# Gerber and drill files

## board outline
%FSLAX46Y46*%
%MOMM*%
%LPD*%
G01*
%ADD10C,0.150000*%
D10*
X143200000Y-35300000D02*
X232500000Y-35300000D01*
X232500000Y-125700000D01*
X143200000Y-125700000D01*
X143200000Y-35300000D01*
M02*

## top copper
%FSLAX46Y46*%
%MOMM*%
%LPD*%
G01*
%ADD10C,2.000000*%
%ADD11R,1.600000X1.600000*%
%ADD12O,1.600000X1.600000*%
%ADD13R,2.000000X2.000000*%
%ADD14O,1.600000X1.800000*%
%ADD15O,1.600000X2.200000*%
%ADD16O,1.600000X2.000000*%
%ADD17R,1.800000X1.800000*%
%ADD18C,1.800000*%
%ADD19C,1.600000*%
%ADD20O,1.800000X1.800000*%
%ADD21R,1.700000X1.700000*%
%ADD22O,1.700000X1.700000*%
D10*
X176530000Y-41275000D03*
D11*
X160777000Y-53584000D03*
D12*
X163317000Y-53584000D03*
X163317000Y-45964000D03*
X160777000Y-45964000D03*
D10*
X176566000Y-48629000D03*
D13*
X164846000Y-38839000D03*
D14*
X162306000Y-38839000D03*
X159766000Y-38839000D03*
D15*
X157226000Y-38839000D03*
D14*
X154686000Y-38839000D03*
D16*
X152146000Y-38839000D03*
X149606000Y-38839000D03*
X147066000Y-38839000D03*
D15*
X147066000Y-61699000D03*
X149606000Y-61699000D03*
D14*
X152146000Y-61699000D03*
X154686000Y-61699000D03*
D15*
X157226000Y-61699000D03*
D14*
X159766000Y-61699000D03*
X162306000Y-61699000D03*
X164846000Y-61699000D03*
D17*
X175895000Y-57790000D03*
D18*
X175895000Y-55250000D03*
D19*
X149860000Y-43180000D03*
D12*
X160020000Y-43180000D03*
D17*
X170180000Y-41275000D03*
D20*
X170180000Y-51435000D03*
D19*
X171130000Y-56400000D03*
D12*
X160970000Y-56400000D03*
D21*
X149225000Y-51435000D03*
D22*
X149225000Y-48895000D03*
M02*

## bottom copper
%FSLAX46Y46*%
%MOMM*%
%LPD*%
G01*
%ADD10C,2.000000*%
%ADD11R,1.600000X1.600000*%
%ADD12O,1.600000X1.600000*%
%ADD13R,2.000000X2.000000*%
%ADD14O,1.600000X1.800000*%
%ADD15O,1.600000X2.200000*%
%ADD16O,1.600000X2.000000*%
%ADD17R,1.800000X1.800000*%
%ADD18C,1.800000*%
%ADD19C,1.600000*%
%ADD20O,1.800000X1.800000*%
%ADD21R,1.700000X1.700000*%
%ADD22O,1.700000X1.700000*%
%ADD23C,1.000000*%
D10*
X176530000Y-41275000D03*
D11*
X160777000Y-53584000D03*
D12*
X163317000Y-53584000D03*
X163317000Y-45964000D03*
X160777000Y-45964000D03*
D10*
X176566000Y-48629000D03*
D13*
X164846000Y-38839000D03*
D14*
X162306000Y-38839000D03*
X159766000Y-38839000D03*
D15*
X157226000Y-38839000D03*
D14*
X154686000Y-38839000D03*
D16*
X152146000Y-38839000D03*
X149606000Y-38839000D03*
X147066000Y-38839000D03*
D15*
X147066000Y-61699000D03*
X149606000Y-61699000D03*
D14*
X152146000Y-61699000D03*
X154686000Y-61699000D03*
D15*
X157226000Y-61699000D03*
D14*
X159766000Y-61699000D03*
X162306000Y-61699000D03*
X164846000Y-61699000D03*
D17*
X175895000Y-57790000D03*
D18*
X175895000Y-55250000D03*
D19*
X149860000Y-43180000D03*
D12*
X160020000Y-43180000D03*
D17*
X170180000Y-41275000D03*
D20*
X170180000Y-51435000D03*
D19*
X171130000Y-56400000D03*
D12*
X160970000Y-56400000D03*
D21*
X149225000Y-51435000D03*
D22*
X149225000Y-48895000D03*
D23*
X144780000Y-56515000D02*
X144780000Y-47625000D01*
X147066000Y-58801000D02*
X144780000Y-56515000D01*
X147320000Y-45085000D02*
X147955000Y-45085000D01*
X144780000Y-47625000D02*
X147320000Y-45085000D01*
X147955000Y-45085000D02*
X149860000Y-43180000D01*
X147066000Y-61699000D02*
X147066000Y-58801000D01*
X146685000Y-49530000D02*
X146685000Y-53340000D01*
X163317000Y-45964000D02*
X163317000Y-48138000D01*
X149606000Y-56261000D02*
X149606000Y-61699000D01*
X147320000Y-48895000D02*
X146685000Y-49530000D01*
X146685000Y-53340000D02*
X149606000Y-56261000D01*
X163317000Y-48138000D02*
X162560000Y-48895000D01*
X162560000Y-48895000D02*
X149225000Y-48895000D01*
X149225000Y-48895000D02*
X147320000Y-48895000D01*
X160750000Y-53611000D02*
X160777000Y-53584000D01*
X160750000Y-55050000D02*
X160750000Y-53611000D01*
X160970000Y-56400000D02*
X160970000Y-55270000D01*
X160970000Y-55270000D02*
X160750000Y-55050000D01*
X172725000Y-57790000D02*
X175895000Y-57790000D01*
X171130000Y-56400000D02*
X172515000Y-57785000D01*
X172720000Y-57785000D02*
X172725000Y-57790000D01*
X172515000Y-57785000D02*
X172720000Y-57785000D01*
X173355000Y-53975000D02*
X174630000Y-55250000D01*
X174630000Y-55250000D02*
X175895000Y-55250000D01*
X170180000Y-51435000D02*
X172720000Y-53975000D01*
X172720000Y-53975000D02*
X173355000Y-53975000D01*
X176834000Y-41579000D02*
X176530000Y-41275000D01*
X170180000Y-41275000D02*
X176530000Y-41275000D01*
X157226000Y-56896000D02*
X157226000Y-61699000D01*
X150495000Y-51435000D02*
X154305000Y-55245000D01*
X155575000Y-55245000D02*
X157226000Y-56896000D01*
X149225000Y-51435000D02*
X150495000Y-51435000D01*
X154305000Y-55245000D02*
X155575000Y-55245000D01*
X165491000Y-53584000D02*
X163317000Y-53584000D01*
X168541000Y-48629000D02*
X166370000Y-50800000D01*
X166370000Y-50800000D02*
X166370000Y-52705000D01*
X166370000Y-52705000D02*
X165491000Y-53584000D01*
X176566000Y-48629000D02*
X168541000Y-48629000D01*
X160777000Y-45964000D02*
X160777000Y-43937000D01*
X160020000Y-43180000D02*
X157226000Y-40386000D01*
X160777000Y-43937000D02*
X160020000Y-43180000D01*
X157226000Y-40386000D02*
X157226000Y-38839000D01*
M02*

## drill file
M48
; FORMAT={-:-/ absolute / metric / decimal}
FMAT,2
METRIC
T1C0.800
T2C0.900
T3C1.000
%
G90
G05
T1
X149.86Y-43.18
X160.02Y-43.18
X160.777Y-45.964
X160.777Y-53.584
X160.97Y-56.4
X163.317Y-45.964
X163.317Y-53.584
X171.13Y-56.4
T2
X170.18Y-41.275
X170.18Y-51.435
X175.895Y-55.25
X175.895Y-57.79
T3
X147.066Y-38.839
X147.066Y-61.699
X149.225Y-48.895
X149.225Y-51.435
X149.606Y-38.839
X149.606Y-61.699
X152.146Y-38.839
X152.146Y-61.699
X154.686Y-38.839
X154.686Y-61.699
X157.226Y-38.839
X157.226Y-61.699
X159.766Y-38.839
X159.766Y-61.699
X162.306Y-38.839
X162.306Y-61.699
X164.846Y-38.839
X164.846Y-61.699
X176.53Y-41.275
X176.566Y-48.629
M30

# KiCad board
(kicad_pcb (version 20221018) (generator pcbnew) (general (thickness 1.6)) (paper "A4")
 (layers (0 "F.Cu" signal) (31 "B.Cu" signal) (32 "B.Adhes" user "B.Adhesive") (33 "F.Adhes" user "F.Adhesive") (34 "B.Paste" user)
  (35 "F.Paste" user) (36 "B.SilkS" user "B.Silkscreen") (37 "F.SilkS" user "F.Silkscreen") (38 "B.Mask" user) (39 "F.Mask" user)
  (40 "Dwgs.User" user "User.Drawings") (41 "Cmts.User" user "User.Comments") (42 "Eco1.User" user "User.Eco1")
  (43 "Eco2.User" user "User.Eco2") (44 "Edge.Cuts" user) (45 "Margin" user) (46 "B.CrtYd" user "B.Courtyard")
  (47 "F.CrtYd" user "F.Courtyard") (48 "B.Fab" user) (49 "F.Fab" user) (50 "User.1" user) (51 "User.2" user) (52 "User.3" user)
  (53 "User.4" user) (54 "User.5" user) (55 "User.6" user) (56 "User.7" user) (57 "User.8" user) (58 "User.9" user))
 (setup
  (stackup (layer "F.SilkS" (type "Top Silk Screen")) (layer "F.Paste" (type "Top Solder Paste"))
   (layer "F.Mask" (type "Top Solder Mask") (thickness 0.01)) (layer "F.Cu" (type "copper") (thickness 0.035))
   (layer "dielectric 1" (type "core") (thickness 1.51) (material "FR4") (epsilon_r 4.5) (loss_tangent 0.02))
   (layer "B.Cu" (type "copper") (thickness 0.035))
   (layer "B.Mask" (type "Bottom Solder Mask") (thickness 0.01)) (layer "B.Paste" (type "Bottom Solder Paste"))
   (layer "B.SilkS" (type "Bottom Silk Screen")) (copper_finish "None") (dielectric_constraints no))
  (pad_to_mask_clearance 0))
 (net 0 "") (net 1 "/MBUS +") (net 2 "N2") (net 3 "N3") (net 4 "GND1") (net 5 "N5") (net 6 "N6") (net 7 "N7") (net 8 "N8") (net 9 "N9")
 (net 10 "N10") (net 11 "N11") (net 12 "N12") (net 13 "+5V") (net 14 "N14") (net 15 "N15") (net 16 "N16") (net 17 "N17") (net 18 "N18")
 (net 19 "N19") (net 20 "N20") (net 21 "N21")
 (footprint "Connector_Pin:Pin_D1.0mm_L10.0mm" (layer "F.Cu") (at 176.53 41.275 180)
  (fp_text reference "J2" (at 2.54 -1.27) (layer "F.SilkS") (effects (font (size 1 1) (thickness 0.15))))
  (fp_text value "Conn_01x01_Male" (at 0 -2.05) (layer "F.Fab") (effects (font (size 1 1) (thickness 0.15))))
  (pad "1" thru_hole circle (at 0 0 180) (size 2 2) (drill 1) (layers "*.Cu" "*.Mask") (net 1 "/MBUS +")))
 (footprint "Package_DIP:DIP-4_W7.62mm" (layer "F.Cu") (at 160.777 53.584 90)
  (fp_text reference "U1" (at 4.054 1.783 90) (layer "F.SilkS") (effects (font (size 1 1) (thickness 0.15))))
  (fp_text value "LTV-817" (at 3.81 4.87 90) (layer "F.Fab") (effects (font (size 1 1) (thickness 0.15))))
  (pad "1" thru_hole rect (at 0 0 90) (size 1.6 1.6) (drill 0.8) (layers "*.Cu" "*.Mask") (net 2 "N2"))
  (pad "2" thru_hole oval (at 0 2.54 90) (size 1.6 1.6) (drill 0.8) (layers "*.Cu" "*.Mask") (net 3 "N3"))
  (pad "3" thru_hole oval (at 7.62 2.54 90) (size 1.6 1.6) (drill 0.8) (layers "*.Cu" "*.Mask") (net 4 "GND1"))
  (pad "4" thru_hole oval (at 7.62 0 90) (size 1.6 1.6) (drill 0.8) (layers "*.Cu" "*.Mask") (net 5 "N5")))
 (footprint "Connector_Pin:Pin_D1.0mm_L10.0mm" (layer "F.Cu") (at 176.566 48.629 180)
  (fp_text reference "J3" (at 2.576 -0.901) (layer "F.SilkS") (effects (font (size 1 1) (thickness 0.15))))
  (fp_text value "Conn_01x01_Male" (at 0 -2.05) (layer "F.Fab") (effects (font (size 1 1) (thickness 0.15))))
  (pad "1" thru_hole circle (at 0 0 180) (size 2 2) (drill 1) (layers "*.Cu" "*.Mask") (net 3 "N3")))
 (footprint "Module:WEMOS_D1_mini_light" (layer "F.Cu") (at 164.846 38.839 -90)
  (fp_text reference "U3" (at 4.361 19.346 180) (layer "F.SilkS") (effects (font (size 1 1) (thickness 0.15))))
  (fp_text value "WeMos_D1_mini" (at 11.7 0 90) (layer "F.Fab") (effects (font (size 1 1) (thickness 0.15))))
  (pad "1" thru_hole rect (at 0 0 270) (size 2 2) (drill 1) (layers "*.Cu" "*.Mask") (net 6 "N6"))
  (pad "2" thru_hole oval (at 0 2.54 270) (size 1.8 1.6) (drill 1) (layers "*.Cu" "*.Mask") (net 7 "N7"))
  (pad "3" thru_hole oval (at 0 5.08 270) (size 1.8 1.6) (drill 1) (layers "*.Cu" "*.Mask") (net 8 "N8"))
  (pad "4" thru_hole oval (at 0 7.62 270) (size 2.2 1.6) (drill 1) (layers "*.Cu" "*.Mask") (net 5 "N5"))
  (pad "5" thru_hole oval (at 0 10.16 270) (size 1.8 1.6) (drill 1) (layers "*.Cu" "*.Mask") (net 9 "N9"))
  (pad "6" thru_hole oval (at 0 12.7 270) (size 2 1.6) (drill 1) (layers "*.Cu" "*.Mask") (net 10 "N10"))
  (pad "7" thru_hole oval (at 0 15.24 270) (size 2 1.6) (drill 1) (layers "*.Cu" "*.Mask") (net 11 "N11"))
  (pad "8" thru_hole oval (at 0 17.78 270) (size 2 1.6) (drill 1) (layers "*.Cu" "*.Mask") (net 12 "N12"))
  (pad "9" thru_hole oval (at 22.86 17.78 270) (size 2.2 1.6) (drill 1) (layers "*.Cu" "*.Mask") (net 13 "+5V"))
  (pad "10" thru_hole oval (at 22.86 15.24 270) (size 2.2 1.6) (drill 1) (layers "*.Cu" "*.Mask") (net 4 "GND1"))
  (pad "11" thru_hole oval (at 22.86 12.7 270) (size 1.8 1.6) (drill 1) (layers "*.Cu" "*.Mask") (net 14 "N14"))
  (pad "12" thru_hole oval (at 22.86 10.16 270) (size 1.8 1.6) (drill 1) (layers "*.Cu" "*.Mask") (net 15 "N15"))
  (pad "13" thru_hole oval (at 22.86 7.62 270) (size 2.2 1.6) (drill 1) (layers "*.Cu" "*.Mask") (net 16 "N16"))
  (pad "14" thru_hole oval (at 22.86 5.08 270) (size 1.8 1.6) (drill 1) (layers "*.Cu" "*.Mask") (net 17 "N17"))
  (pad "15" thru_hole oval (at 22.86 2.54 270) (size 1.8 1.6) (drill 1) (layers "*.Cu" "*.Mask") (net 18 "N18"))
  (pad "16" thru_hole oval (at 22.86 0 270) (size 1.8 1.6) (drill 1) (layers "*.Cu" "*.Mask") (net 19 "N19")))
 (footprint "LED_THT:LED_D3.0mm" (layer "F.Cu") (at 175.895 57.79 90)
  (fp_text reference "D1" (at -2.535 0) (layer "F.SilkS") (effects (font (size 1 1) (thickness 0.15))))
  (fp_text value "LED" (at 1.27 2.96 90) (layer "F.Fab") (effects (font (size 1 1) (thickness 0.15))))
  (pad "1" thru_hole rect (at 0 0 90) (size 1.8 1.8) (drill 0.9) (layers "*.Cu" "*.Mask") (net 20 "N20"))
  (pad "2" thru_hole circle (at 2.54 0 90) (size 1.8 1.8) (drill 0.9) (layers "*.Cu" "*.Mask") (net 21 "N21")))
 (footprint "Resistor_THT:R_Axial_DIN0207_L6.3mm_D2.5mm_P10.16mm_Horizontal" (layer "F.Cu") (at 149.86 43.18)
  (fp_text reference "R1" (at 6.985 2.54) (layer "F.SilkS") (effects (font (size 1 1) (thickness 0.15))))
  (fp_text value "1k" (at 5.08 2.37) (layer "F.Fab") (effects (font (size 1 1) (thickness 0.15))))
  (pad "1" thru_hole circle (at 0 0) (size 1.6 1.6) (drill 0.8) (layers "*.Cu" "*.Mask") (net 13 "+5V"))
  (pad "2" thru_hole oval (at 10.16 0) (size 1.6 1.6) (drill 0.8) (layers "*.Cu" "*.Mask") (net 5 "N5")))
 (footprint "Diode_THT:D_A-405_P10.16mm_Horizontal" (layer "F.Cu") (at 170.18 41.275 -90)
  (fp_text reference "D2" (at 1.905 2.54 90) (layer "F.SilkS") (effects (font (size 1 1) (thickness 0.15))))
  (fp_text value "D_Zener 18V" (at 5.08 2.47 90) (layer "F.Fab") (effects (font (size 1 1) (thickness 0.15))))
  (pad "1" thru_hole rect (at 0 0 270) (size 1.8 1.8) (drill 0.9) (layers "*.Cu" "*.Mask") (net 1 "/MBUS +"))
  (pad "2" thru_hole oval (at 10.16 0 270) (size 1.8 1.8) (drill 0.9) (layers "*.Cu" "*.Mask") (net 21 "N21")))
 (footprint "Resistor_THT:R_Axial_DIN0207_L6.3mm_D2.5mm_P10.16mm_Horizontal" (layer "F.Cu") (at 171.13 56.4 180)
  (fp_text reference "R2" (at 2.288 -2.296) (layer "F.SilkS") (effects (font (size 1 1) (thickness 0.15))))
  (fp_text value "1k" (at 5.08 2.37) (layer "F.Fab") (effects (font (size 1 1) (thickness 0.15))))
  (pad "1" thru_hole circle (at 0 0 180) (size 1.6 1.6) (drill 0.8) (layers "*.Cu" "*.Mask") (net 20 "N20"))
  (pad "2" thru_hole oval (at 10.16 0 180) (size 1.6 1.6) (drill 0.8) (layers "*.Cu" "*.Mask") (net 2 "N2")))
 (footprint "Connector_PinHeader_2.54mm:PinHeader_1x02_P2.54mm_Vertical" (layer "F.Cu") (at 149.225 51.435 180)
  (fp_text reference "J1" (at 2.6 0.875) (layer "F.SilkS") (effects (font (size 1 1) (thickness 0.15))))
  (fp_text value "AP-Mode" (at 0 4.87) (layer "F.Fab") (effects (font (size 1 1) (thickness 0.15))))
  (pad "1" thru_hole rect (at 0 0 180) (size 1.7 1.7) (drill 1) (layers "*.Cu" "*.Mask") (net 16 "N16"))
  (pad "2" thru_hole oval (at 0 2.54 180) (size 1.7 1.7) (drill 1) (layers "*.Cu" "*.Mask") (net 4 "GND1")))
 (gr_rect (start 143.2 35.3) (end 232.5 125.7) (stroke (width 0.15) (type solid)) (fill none) (layer "Edge.Cuts"))
 (segment (start 144.78 56.515) (end 144.78 47.625) (width 1) (layer "B.Cu") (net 13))
 (segment (start 147.066 58.801) (end 144.78 56.515) (width 1) (layer "B.Cu") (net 13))
 (segment (start 147.32 45.085) (end 147.955 45.085) (width 1) (layer "B.Cu") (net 13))
 (segment (start 144.78 47.625) (end 147.32 45.085) (width 1) (layer "B.Cu") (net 13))
 (segment (start 147.955 45.085) (end 149.86 43.18) (width 1) (layer "B.Cu") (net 13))
 (segment (start 147.066 61.699) (end 147.066 58.801) (width 1) (layer "B.Cu") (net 13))
 (segment (start 146.685 49.53) (end 146.685 53.34) (width 1) (layer "B.Cu") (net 4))
 (segment (start 163.317 45.964) (end 163.317 48.138) (width 1) (layer "B.Cu") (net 4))
 (segment (start 149.606 56.261) (end 149.606 61.699) (width 1) (layer "B.Cu") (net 4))
 (segment (start 147.32 48.895) (end 146.685 49.53) (width 1) (layer "B.Cu") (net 4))
 (segment (start 146.685 53.34) (end 149.606 56.261) (width 1) (layer "B.Cu") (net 4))
 (segment (start 163.317 48.138) (end 162.56 48.895) (width 1) (layer "B.Cu") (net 4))
 (segment (start 162.56 48.895) (end 149.225 48.895) (width 1) (layer "B.Cu") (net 4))
 (segment (start 149.225 48.895) (end 147.32 48.895) (width 1) (layer "B.Cu") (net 4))
 (segment (start 160.75 53.611) (end 160.777 53.584) (width 1) (layer "B.Cu") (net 2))
 (segment (start 160.75 55.05) (end 160.75 53.611) (width 1) (layer "B.Cu") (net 2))
 (segment (start 160.97 56.4) (end 160.97 55.27) (width 1) (layer "B.Cu") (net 2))
 (segment (start 160.97 55.27) (end 160.75 55.05) (width 1) (layer "B.Cu") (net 2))
 (segment (start 172.725 57.79) (end 175.895 57.79) (width 1) (layer "B.Cu") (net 20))
 (segment (start 171.13 56.4) (end 172.515 57.785) (width 1) (layer "B.Cu") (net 20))
 (segment (start 172.72 57.785) (end 172.725 57.79) (width 1) (layer "B.Cu") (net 20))
 (segment (start 172.515 57.785) (end 172.72 57.785) (width 1) (layer "B.Cu") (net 20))
 (segment (start 173.355 53.975) (end 174.63 55.25) (width 1) (layer "B.Cu") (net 21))
 (segment (start 174.63 55.25) (end 175.895 55.25) (width 1) (layer "B.Cu") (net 21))
 (segment (start 170.18 51.435) (end 172.72 53.975) (width 1) (layer "B.Cu") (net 21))
 (segment (start 172.72 53.975) (end 173.355 53.975) (width 1) (layer "B.Cu") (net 21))
 (segment (start 176.834 41.579) (end 176.53 41.275) (width 1) (layer "B.Cu") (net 1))
 (segment (start 170.18 41.275) (end 176.53 41.275) (width 1) (layer "B.Cu") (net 1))
 (segment (start 157.226 56.896) (end 157.226 61.699) (width 1) (layer "B.Cu") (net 16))
 (segment (start 150.495 51.435) (end 154.305 55.245) (width 1) (layer "B.Cu") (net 16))
 (segment (start 155.575 55.245) (end 157.226 56.896) (width 1) (layer "B.Cu") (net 16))
 (segment (start 149.225 51.435) (end 150.495 51.435) (width 1) (layer "B.Cu") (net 16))
 (segment (start 154.305 55.245) (end 155.575 55.245) (width 1) (layer "B.Cu") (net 16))
 (segment (start 165.491 53.584) (end 163.317 53.584) (width 1) (layer "B.Cu") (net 3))
 (segment (start 168.541 48.629) (end 166.37 50.8) (width 1) (layer "B.Cu") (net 3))
 (segment (start 166.37 50.8) (end 166.37 52.705) (width 1) (layer "B.Cu") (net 3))
 (segment (start 166.37 52.705) (end 165.491 53.584) (width 1) (layer "B.Cu") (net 3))
 (segment (start 176.566 48.629) (end 168.541 48.629) (width 1) (layer "B.Cu") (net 3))
 (segment (start 160.777 45.964) (end 160.777 43.937) (width 1) (layer "B.Cu") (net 5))
 (segment (start 160.02 43.18) (end 157.226 40.386) (width 1) (layer "B.Cu") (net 5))
 (segment (start 160.777 43.937) (end 160.02 43.18) (width 1) (layer "B.Cu") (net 5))
 (segment (start 157.226 40.386) (end 157.226 38.839) (width 1) (layer "B.Cu") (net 5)))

